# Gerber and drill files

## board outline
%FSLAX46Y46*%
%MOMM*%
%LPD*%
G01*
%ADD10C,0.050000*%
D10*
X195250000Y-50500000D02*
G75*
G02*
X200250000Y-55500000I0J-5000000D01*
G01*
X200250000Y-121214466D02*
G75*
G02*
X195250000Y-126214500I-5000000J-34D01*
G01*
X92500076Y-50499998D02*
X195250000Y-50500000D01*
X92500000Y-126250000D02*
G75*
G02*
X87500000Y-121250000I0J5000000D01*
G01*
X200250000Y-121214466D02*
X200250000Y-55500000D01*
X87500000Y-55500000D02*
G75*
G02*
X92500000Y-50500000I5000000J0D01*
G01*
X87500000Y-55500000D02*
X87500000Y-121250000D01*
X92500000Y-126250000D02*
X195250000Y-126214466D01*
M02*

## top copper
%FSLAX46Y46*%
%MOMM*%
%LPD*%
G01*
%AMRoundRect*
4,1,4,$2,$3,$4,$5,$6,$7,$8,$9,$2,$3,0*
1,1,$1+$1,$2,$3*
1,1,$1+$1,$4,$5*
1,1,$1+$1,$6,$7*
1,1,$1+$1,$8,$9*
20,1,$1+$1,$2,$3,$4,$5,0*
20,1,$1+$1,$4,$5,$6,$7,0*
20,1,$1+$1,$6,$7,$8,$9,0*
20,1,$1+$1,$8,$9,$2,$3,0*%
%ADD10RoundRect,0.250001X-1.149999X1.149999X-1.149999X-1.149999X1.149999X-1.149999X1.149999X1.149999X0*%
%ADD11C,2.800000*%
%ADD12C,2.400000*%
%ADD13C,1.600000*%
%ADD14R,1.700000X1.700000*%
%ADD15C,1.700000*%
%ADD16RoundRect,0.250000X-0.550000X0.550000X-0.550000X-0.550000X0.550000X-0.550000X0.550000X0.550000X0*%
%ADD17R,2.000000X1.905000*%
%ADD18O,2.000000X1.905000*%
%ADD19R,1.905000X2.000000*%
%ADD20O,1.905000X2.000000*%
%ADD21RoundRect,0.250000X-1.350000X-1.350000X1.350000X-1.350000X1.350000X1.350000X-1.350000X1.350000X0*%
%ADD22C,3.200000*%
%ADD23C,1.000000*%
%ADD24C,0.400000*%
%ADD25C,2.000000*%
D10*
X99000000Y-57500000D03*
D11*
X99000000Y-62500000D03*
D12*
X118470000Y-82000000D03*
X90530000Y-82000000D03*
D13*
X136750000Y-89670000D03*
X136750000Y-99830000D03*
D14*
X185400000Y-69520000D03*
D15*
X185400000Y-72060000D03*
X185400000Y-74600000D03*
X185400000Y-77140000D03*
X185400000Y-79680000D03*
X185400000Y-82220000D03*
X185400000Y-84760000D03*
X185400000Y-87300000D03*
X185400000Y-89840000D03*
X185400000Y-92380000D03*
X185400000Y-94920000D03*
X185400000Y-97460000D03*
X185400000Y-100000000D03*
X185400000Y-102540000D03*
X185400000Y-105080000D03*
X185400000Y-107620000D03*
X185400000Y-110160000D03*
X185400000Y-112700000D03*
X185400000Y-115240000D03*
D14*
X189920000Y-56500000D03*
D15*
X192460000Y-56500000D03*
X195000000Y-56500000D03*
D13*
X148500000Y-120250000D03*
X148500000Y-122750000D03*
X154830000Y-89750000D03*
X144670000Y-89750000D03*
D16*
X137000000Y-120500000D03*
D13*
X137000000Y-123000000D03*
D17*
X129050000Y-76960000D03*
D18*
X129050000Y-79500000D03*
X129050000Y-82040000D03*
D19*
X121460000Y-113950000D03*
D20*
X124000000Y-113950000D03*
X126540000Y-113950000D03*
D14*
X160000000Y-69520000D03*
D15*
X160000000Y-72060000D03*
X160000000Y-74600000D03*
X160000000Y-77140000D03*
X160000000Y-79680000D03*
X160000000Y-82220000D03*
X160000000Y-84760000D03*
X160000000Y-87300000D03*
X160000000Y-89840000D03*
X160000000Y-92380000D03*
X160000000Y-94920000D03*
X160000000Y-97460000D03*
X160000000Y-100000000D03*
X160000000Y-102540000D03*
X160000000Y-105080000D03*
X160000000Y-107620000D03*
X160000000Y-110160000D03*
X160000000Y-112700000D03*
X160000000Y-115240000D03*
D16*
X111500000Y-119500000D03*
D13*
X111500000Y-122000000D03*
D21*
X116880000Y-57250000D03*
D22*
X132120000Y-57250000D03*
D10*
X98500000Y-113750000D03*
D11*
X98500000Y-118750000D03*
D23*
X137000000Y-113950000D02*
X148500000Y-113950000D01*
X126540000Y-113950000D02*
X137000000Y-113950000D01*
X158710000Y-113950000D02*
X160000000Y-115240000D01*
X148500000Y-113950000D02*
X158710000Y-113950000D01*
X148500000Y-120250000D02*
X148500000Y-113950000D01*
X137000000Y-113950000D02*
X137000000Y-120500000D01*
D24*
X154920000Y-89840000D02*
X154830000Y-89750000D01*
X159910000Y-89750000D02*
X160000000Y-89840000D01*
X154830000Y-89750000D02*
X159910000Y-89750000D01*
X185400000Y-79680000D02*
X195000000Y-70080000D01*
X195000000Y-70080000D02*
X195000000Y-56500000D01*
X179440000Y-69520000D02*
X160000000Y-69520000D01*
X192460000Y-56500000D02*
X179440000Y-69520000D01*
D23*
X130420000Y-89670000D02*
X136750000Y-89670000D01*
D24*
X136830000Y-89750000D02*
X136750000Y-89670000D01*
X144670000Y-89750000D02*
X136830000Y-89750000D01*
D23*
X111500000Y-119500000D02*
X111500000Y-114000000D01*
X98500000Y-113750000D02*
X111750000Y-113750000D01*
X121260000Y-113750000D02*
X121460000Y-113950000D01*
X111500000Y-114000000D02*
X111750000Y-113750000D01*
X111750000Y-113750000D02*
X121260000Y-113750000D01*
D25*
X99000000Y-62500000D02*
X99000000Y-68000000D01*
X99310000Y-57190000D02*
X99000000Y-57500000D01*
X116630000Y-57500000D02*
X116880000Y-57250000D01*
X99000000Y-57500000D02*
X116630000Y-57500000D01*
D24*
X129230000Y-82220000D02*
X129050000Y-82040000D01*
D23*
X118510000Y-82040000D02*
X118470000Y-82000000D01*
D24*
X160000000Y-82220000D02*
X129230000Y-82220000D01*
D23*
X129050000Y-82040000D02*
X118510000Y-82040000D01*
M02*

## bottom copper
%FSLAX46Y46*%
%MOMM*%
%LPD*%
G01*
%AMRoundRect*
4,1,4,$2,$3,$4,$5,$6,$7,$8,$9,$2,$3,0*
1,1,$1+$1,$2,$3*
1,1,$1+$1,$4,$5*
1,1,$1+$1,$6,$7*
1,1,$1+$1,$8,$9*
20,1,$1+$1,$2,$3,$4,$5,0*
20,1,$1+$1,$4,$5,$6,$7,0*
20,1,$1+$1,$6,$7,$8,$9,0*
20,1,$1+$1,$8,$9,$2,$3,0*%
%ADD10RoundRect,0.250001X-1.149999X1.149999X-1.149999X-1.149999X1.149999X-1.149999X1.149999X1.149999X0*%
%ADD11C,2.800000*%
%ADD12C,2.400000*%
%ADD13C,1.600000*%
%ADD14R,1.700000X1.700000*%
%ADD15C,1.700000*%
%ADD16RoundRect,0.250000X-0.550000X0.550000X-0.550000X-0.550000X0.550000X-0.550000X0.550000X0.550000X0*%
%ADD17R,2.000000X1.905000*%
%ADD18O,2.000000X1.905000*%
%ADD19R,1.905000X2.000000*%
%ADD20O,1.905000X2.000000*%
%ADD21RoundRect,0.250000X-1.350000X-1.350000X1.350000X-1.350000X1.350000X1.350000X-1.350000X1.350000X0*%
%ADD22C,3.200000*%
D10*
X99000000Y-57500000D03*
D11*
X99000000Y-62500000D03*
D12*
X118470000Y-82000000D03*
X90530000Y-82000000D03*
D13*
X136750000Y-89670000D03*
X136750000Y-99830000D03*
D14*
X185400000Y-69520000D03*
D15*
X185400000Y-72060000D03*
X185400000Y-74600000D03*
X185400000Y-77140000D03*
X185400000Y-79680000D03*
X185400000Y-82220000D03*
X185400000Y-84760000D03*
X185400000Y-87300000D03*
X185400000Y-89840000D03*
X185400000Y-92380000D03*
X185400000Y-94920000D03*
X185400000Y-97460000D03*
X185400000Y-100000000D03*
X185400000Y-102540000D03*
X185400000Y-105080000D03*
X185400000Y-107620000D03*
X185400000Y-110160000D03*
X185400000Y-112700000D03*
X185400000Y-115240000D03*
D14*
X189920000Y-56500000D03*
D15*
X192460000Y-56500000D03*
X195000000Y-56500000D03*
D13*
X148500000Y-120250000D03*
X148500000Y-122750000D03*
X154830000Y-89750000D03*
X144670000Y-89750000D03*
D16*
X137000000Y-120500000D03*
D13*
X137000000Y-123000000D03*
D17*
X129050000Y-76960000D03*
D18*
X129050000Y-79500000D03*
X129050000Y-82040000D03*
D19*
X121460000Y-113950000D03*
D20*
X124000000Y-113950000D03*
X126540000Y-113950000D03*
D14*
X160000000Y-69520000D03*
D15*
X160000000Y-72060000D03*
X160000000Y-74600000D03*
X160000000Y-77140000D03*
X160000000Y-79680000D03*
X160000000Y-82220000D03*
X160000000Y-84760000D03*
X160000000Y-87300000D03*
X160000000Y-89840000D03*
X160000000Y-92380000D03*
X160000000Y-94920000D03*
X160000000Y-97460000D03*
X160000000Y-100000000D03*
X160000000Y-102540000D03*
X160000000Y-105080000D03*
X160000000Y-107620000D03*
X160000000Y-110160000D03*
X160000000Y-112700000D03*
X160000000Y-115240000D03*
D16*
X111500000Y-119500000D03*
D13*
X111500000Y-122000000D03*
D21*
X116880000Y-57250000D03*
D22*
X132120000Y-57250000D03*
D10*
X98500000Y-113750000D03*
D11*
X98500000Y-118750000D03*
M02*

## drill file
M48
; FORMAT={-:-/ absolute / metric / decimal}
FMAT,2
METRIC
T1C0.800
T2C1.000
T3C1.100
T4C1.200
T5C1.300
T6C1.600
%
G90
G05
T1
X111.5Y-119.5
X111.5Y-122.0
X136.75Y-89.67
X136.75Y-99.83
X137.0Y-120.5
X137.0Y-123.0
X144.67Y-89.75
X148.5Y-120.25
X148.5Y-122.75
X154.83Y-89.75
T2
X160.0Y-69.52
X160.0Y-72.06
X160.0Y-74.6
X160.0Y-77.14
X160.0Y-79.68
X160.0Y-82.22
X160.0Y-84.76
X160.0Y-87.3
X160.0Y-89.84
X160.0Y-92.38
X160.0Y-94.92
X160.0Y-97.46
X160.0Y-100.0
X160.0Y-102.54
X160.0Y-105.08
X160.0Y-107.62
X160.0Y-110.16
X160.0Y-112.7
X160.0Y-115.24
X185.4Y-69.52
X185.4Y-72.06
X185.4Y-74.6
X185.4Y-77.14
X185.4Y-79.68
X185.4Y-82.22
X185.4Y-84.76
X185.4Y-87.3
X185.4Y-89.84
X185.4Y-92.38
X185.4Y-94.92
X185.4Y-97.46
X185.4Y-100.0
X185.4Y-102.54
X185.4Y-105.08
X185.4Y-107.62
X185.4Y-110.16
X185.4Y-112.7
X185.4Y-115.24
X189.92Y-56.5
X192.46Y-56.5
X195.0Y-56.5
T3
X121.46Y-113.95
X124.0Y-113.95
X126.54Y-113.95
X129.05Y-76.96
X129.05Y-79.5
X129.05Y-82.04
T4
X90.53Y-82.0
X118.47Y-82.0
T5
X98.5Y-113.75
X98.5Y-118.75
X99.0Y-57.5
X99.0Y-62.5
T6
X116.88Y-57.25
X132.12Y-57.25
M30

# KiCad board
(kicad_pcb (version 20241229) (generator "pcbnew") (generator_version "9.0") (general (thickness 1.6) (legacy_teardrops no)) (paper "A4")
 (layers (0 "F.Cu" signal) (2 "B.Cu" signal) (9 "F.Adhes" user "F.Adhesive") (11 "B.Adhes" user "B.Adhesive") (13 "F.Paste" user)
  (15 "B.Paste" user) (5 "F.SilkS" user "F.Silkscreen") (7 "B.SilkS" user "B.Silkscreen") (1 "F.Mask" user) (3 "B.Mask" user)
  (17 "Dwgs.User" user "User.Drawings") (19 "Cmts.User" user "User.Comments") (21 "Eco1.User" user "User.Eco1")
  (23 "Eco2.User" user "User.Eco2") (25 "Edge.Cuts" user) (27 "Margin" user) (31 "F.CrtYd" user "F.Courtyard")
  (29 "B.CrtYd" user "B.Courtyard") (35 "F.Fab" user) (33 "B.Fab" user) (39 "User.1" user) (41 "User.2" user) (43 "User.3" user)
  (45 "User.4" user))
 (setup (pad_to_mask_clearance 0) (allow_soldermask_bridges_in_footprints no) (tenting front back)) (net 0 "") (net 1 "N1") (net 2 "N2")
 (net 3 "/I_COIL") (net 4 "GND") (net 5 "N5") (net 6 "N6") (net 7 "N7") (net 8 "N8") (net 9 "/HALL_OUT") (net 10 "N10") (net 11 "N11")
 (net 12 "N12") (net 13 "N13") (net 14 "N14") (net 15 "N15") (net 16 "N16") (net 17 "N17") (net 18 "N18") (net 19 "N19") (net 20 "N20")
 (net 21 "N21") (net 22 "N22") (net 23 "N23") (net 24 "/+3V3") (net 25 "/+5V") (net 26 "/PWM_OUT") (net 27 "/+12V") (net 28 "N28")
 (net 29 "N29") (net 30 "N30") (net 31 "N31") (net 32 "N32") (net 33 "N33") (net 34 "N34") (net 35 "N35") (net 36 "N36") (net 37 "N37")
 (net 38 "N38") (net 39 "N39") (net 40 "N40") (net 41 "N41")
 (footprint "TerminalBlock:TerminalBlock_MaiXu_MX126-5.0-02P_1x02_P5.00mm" (layer "F.Cu") (at 99 57.5 -90)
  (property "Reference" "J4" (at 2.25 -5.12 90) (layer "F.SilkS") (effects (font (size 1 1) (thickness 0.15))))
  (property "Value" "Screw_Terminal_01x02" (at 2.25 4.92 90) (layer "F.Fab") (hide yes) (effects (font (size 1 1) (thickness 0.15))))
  (pad "1" thru_hole roundrect (at 0 0 270) (size 2.8 2.8) (drill 1.3) (layers "*.Cu" "*.Mask") (remove_unused_layers no)
   (roundrect_rratio 0.089286) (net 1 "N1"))
  (pad "2" thru_hole circle (at 5 0 270) (size 2.8 2.8) (drill 1.3) (layers "*.Cu" "*.Mask") (remove_unused_layers no) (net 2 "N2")))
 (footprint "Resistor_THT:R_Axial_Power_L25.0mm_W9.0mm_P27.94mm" (layer "F.Cu") (at 118.47 82 180)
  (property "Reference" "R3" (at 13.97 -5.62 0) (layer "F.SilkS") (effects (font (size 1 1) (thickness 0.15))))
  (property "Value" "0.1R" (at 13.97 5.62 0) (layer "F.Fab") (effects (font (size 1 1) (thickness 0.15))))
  (pad "1" thru_hole circle (at 0 0 180) (size 2.4 2.4) (drill 1.2) (layers "*.Cu" "*.Mask") (remove_unused_layers no) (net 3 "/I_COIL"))
  (pad "2" thru_hole circle (at 27.94 0 180) (size 2.4 2.4) (drill 1.2) (layers "*.Cu" "*.Mask") (remove_unused_layers no) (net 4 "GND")))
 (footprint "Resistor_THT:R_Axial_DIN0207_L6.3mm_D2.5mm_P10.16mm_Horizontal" (layer "F.Cu") (at 136.75 89.67 -90)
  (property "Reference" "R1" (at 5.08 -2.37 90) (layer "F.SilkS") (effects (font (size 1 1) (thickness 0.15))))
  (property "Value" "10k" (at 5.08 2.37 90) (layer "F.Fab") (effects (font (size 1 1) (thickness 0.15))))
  (pad "1" thru_hole circle (at 0 0 270) (size 1.6 1.6) (drill 0.8) (layers "*.Cu" "*.Mask") (remove_unused_layers no) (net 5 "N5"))
  (pad "2" thru_hole circle (at 10.16 0 270) (size 1.6 1.6) (drill 0.8) (layers "*.Cu" "*.Mask") (remove_unused_layers no) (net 4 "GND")))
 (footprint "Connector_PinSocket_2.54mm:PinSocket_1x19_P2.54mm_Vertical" (layer "F.Cu") (at 185.4 69.52)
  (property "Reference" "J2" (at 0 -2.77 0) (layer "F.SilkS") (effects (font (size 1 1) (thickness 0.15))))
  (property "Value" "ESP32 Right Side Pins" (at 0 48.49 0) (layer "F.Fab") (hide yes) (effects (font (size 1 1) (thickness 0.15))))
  (pad "1" thru_hole rect (at 0 0) (size 1.7 1.7) (drill 1) (layers "*.Cu" "*.Mask") (remove_unused_layers no) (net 4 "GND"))
  (pad "2" thru_hole circle (at 0 2.54) (size 1.7 1.7) (drill 1) (layers "*.Cu" "*.Mask") (remove_unused_layers no) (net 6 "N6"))
  (pad "3" thru_hole circle (at 0 5.08) (size 1.7 1.7) (drill 1) (layers "*.Cu" "*.Mask") (remove_unused_layers no) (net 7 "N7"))
  (pad "4" thru_hole circle (at 0 7.62) (size 1.7 1.7) (drill 1) (layers "*.Cu" "*.Mask") (remove_unused_layers no) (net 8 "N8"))
  (pad "5" thru_hole circle (at 0 10.16) (size 1.7 1.7) (drill 1) (layers "*.Cu" "*.Mask") (remove_unused_layers no) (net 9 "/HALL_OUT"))
  (pad "6" thru_hole circle (at 0 12.7) (size 1.7 1.7) (drill 1) (layers "*.Cu" "*.Mask") (remove_unused_layers no) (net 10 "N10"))
  (pad "7" thru_hole circle (at 0 15.24) (size 1.7 1.7) (drill 1) (layers "*.Cu" "*.Mask") (remove_unused_layers no) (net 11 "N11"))
  (pad "8" thru_hole circle (at 0 17.78) (size 1.7 1.7) (drill 1) (layers "*.Cu" "*.Mask") (remove_unused_layers no) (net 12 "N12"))
  (pad "9" thru_hole circle (at 0 20.32) (size 1.7 1.7) (drill 1) (layers "*.Cu" "*.Mask") (remove_unused_layers no) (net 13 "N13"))
  (pad "10" thru_hole circle (at 0 22.86) (size 1.7 1.7) (drill 1) (layers "*.Cu" "*.Mask") (remove_unused_layers no) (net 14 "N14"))
  (pad "11" thru_hole circle (at 0 25.4) (size 1.7 1.7) (drill 1) (layers "*.Cu" "*.Mask") (remove_unused_layers no) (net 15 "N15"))
  (pad "12" thru_hole circle (at 0 27.94) (size 1.7 1.7) (drill 1) (layers "*.Cu" "*.Mask") (remove_unused_layers no) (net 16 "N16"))
  (pad "13" thru_hole circle (at 0 30.48) (size 1.7 1.7) (drill 1) (layers "*.Cu" "*.Mask") (remove_unused_layers no) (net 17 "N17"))
  (pad "14" thru_hole circle (at 0 33.02) (size 1.7 1.7) (drill 1) (layers "*.Cu" "*.Mask") (remove_unused_layers no) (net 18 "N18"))
  (pad "15" thru_hole circle (at 0 35.56) (size 1.7 1.7) (drill 1) (layers "*.Cu" "*.Mask") (remove_unused_layers no) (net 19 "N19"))
  (pad "16" thru_hole circle (at 0 38.1) (size 1.7 1.7) (drill 1) (layers "*.Cu" "*.Mask") (remove_unused_layers no) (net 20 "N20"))
  (pad "17" thru_hole circle (at 0 40.64) (size 1.7 1.7) (drill 1) (layers "*.Cu" "*.Mask") (remove_unused_layers no) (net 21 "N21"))
  (pad "18" thru_hole circle (at 0 43.18) (size 1.7 1.7) (drill 1) (layers "*.Cu" "*.Mask") (remove_unused_layers no) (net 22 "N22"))
  (pad "19" thru_hole circle (at 0 45.72) (size 1.7 1.7) (drill 1) (layers "*.Cu" "*.Mask") (remove_unused_layers no) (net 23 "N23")))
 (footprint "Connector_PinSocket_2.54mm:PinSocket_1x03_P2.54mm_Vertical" (layer "F.Cu") (at 189.92 56.5 90)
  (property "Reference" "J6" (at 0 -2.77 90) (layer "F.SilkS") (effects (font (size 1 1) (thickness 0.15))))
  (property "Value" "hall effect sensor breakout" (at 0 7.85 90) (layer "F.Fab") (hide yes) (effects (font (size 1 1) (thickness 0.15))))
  (pad "1" thru_hole rect (at 0 0 90) (size 1.7 1.7) (drill 1) (layers "*.Cu" "*.Mask") (remove_unused_layers no) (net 4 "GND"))
  (pad "2" thru_hole circle (at 0 2.54 90) (size 1.7 1.7) (drill 1) (layers "*.Cu" "*.Mask") (remove_unused_layers no) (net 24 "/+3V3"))
  (pad "3" thru_hole circle (at 0 5.08 90) (size 1.7 1.7) (drill 1) (layers "*.Cu" "*.Mask") (remove_unused_layers no) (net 9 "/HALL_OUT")))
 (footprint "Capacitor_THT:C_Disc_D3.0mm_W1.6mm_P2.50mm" (layer "F.Cu") (at 148.5 120.25 -90)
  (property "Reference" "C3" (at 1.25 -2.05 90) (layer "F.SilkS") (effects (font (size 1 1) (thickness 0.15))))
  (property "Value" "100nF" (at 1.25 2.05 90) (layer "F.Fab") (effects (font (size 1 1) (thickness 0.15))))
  (pad "1" thru_hole circle (at 0 0 270) (size 1.6 1.6) (drill 0.8) (layers "*.Cu" "*.Mask") (remove_unused_layers no) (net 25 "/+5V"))
  (pad "2" thru_hole circle (at 2.5 0 270) (size 1.6 1.6) (drill 0.8) (layers "*.Cu" "*.Mask") (remove_unused_layers no) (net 4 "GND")))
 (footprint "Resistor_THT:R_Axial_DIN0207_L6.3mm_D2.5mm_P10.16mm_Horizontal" (layer "F.Cu") (at 154.83 89.75 180)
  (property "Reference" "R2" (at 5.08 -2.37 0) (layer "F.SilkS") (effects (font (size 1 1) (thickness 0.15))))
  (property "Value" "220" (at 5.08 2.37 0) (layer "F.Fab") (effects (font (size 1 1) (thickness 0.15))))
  (pad "1" thru_hole circle (at 0 0 180) (size 1.6 1.6) (drill 0.8) (layers "*.Cu" "*.Mask") (remove_unused_layers no) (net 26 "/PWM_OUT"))
  (pad "2" thru_hole circle (at 10.16 0 180) (size 1.6 1.6) (drill 0.8) (layers "*.Cu" "*.Mask") (remove_unused_layers no) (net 5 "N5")))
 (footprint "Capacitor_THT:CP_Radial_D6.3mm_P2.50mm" (layer "F.Cu") (at 137 120.5 -90)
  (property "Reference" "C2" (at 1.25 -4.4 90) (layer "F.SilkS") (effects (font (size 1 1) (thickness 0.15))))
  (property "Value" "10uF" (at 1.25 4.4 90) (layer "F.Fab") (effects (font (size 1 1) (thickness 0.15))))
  (pad "1" thru_hole roundrect (at 0 0 270) (size 1.6 1.6) (drill 0.8) (layers "*.Cu" "*.Mask") (remove_unused_layers no)
   (roundrect_rratio 0.15625) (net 25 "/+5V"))
  (pad "2" thru_hole circle (at 2.5 0 270) (size 1.6 1.6) (drill 0.8) (layers "*.Cu" "*.Mask") (remove_unused_layers no) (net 4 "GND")))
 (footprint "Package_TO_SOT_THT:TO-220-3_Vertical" (layer "F.Cu") (at 129.05 76.96 -90)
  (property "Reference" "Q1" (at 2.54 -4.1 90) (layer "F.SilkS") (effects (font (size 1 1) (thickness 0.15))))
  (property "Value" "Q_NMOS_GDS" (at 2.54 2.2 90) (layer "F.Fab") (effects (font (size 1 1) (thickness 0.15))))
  (pad "1" thru_hole rect (at 0 0 270) (size 1.905 2) (drill 1.1) (layers "*.Cu" "*.Mask") (remove_unused_layers no) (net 5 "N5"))
  (pad "2" thru_hole oval (at 2.54 0 270) (size 1.905 2) (drill 1.1) (layers "*.Cu" "*.Mask") (remove_unused_layers no) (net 2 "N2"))
  (pad "3" thru_hole oval (at 5.08 0 270) (size 1.905 2) (drill 1.1) (layers "*.Cu" "*.Mask") (remove_unused_layers no) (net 3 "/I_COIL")))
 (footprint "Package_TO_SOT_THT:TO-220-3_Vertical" (layer "F.Cu") (at 121.46 113.95)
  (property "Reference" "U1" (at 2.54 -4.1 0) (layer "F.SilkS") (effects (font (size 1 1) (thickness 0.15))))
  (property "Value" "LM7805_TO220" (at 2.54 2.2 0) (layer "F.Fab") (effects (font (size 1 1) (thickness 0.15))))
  (pad "1" thru_hole rect (at 0 0) (size 1.905 2) (drill 1.1) (layers "*.Cu" "*.Mask") (remove_unused_layers no) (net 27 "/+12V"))
  (pad "2" thru_hole oval (at 2.54 0) (size 1.905 2) (drill 1.1) (layers "*.Cu" "*.Mask") (remove_unused_layers no) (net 4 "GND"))
  (pad "3" thru_hole oval (at 5.08 0) (size 1.905 2) (drill 1.1) (layers "*.Cu" "*.Mask") (remove_unused_layers no) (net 25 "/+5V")))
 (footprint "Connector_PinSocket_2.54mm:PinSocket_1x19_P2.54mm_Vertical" (layer "F.Cu") (at 160 69.52)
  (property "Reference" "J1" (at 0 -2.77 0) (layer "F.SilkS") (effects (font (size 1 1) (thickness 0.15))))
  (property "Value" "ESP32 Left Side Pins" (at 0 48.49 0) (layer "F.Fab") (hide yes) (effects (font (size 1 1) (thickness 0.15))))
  (pad "1" thru_hole rect (at 0 0) (size 1.7 1.7) (drill 1) (layers "*.Cu" "*.Mask") (remove_unused_layers no) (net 24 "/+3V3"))
  (pad "2" thru_hole circle (at 0 2.54) (size 1.7 1.7) (drill 1) (layers "*.Cu" "*.Mask") (remove_unused_layers no) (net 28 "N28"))
  (pad "3" thru_hole circle (at 0 5.08) (size 1.7 1.7) (drill 1) (layers "*.Cu" "*.Mask") (remove_unused_layers no) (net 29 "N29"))
  (pad "4" thru_hole circle (at 0 7.62) (size 1.7 1.7) (drill 1) (layers "*.Cu" "*.Mask") (remove_unused_layers no) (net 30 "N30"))
  (pad "5" thru_hole circle (at 0 10.16) (size 1.7 1.7) (drill 1) (layers "*.Cu" "*.Mask") (remove_unused_layers no) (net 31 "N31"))
  (pad "6" thru_hole circle (at 0 12.7) (size 1.7 1.7) (drill 1) (layers "*.Cu" "*.Mask") (remove_unused_layers no) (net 3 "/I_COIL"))
  (pad "7" thru_hole circle (at 0 15.24) (size 1.7 1.7) (drill 1) (layers "*.Cu" "*.Mask") (remove_unused_layers no) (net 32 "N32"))
  (pad "8" thru_hole circle (at 0 17.78) (size 1.7 1.7) (drill 1) (layers "*.Cu" "*.Mask") (remove_unused_layers no) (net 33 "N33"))
  (pad "9" thru_hole circle (at 0 20.32) (size 1.7 1.7) (drill 1) (layers "*.Cu" "*.Mask") (remove_unused_layers no) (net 26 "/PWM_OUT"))
  (pad "10" thru_hole circle (at 0 22.86) (size 1.7 1.7) (drill 1) (layers "*.Cu" "*.Mask") (remove_unused_layers no) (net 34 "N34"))
  (pad "11" thru_hole circle (at 0 25.4) (size 1.7 1.7) (drill 1) (layers "*.Cu" "*.Mask") (remove_unused_layers no) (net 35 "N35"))
  (pad "12" thru_hole circle (at 0 27.94) (size 1.7 1.7) (drill 1) (layers "*.Cu" "*.Mask") (remove_unused_layers no) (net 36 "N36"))
  (pad "13" thru_hole circle (at 0 30.48) (size 1.7 1.7) (drill 1) (layers "*.Cu" "*.Mask") (remove_unused_layers no) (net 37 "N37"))
  (pad "14" thru_hole circle (at 0 33.02) (size 1.7 1.7) (drill 1) (layers "*.Cu" "*.Mask") (remove_unused_layers no) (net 4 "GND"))
  (pad "15" thru_hole circle (at 0 35.56) (size 1.7 1.7) (drill 1) (layers "*.Cu" "*.Mask") (remove_unused_layers no) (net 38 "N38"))
  (pad "16" thru_hole circle (at 0 38.1) (size 1.7 1.7) (drill 1) (layers "*.Cu" "*.Mask") (remove_unused_layers no) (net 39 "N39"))
  (pad "17" thru_hole circle (at 0 40.64) (size 1.7 1.7) (drill 1) (layers "*.Cu" "*.Mask") (remove_unused_layers no) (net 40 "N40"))
  (pad "18" thru_hole circle (at 0 43.18) (size 1.7 1.7) (drill 1) (layers "*.Cu" "*.Mask") (remove_unused_layers no) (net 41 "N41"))
  (pad "19" thru_hole circle (at 0 45.72) (size 1.7 1.7) (drill 1) (layers "*.Cu" "*.Mask") (remove_unused_layers no) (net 25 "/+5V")))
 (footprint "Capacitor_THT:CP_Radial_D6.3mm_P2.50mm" (layer "F.Cu") (at 111.5 119.5 -90)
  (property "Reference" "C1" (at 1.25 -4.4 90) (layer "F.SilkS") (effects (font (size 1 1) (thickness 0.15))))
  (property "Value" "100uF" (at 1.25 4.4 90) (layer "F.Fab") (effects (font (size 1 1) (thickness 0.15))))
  (pad "1" thru_hole roundrect (at 0 0 270) (size 1.6 1.6) (drill 0.8) (layers "*.Cu" "*.Mask") (remove_unused_layers no)
   (roundrect_rratio 0.15625) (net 27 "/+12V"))
  (pad "2" thru_hole circle (at 2.5 0 270) (size 1.6 1.6) (drill 0.8) (layers "*.Cu" "*.Mask") (remove_unused_layers no) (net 4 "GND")))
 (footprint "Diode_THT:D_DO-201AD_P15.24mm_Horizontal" (layer "F.Cu") (at 116.88 57.25)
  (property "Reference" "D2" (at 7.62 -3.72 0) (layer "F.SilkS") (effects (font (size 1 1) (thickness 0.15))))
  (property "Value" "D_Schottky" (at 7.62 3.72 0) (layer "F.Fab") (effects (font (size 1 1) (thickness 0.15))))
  (pad "1" thru_hole roundrect (at 0 0) (size 3.2 3.2) (drill 1.6) (layers "*.Cu" "*.Mask") (remove_unused_layers no)
   (roundrect_rratio 0.078125) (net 1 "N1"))
  (pad "2" thru_hole circle (at 15.24 0) (size 3.2 3.2) (drill 1.6) (layers "*.Cu" "*.Mask") (remove_unused_layers no) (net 2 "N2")))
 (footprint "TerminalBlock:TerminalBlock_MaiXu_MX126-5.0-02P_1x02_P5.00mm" (layer "F.Cu") (at 98.5 113.75 -90)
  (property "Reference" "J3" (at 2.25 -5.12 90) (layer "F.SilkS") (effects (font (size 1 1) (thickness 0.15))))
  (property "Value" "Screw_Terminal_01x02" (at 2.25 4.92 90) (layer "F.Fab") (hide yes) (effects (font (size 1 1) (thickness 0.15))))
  (pad "1" thru_hole roundrect (at 0 0 270) (size 2.8 2.8) (drill 1.3) (layers "*.Cu" "*.Mask") (remove_unused_layers no)
   (roundrect_rratio 0.089286) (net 27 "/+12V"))
  (pad "2" thru_hole circle (at 5 0 270) (size 2.8 2.8) (drill 1.3) (layers "*.Cu" "*.Mask") (remove_unused_layers no) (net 4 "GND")))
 (gr_arc (start 195.25 50.5) (mid 198.785534 51.964466) (end 200.25 55.5) (stroke (width 0.05) (type default)) (layer "Edge.Cuts"))
 (gr_arc (start 200.25 121.214466) (mid 198.785534 124.75) (end 195.25 126.214466) (stroke (width 0.05) (type default)) (layer "Edge.Cuts"))
 (gr_line (start 92.500076 50.499998) (end 195.25 50.5) (stroke (width 0.05) (type default)) (layer "Edge.Cuts"))
 (gr_arc (start 92.5 126.25) (mid 88.964466 124.785534) (end 87.5 121.25) (stroke (width 0.05) (type default)) (layer "Edge.Cuts"))
 (gr_line (start 200.25 121.214466) (end 200.25 55.5) (stroke (width 0.05) (type default)) (layer "Edge.Cuts"))
 (gr_arc (start 87.5 55.5) (mid 88.964466 51.964466) (end 92.5 50.5) (stroke (width 0.05) (type default)) (layer "Edge.Cuts"))
 (gr_line (start 87.5 55.5) (end 87.5 121.25) (stroke (width 0.05) (type default)) (layer "Edge.Cuts"))
 (gr_line (start 92.5 126.25) (end 195.25 126.214466) (stroke (width 0.05) (type default)) (layer "Edge.Cuts"))
 (segment (start 137 113.95) (end 148.5 113.95) (width 1) (layer "F.Cu") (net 25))
 (segment (start 126.54 113.95) (end 137 113.95) (width 1) (layer "F.Cu") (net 25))
 (segment (start 158.71 113.95) (end 160 115.24) (width 1) (layer "F.Cu") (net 25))
 (segment (start 148.5 113.95) (end 158.71 113.95) (width 1) (layer "F.Cu") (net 25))
 (segment (start 148.5 120.25) (end 148.5 113.95) (width 1) (layer "F.Cu") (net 25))
 (segment (start 137 113.95) (end 137 120.5) (width 1) (layer "F.Cu") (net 25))
 (segment (start 154.92 89.84) (end 154.83 89.75) (width 0.4) (layer "F.Cu") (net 26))
 (segment (start 159.91 89.75) (end 160 89.84) (width 0.4) (layer "F.Cu") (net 26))
 (segment (start 154.83 89.75) (end 159.91 89.75) (width 0.4) (layer "F.Cu") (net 26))
 (segment (start 185.4 79.68) (end 195 70.08) (width 0.4) (layer "F.Cu") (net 9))
 (segment (start 195 70.08) (end 195 56.5) (width 0.4) (layer "F.Cu") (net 9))
 (segment (start 179.44 69.52) (end 160 69.52) (width 0.4) (layer "F.Cu") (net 24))
 (segment (start 192.46 56.5) (end 179.44 69.52) (width 0.4) (layer "F.Cu") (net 24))
 (segment (start 130.42 89.67) (end 136.75 89.67) (width 1) (layer "F.Cu") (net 5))
 (segment (start 136.83 89.75) (end 136.75 89.67) (width 0.4) (layer "F.Cu") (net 5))
 (segment (start 144.67 89.75) (end 136.83 89.75) (width 0.4) (layer "F.Cu") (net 5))
 (segment (start 111.5 119.5) (end 111.5 114) (width 1) (layer "F.Cu") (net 27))
 (segment (start 98.5 113.75) (end 111.75 113.75) (width 1) (layer "F.Cu") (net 27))
 (segment (start 121.26 113.75) (end 121.46 113.95) (width 1) (layer "F.Cu") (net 27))
 (segment (start 111.5 114) (end 111.75 113.75) (width 1) (layer "F.Cu") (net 27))
 (segment (start 111.75 113.75) (end 121.26 113.75) (width 1) (layer "F.Cu") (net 27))
 (segment (start 99 62.5) (end 99 68) (width 2) (layer "F.Cu") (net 2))
 (segment (start 99.31 57.19) (end 99 57.5) (width 2) (layer "F.Cu") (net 1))
 (segment (start 116.63 57.5) (end 116.88 57.25) (width 2) (layer "F.Cu") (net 1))
 (segment (start 99 57.5) (end 116.63 57.5) (width 2) (layer "F.Cu") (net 1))
 (segment (start 129.23 82.22) (end 129.05 82.04) (width 0.4) (layer "F.Cu") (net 3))
 (segment (start 118.51 82.04) (end 118.47 82) (width 1) (layer "F.Cu") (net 3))
 (segment (start 160 82.22) (end 129.23 82.22) (width 0.4) (layer "F.Cu") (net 3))
 (segment (start 129.05 82.04) (end 118.51 82.04) (width 1) (layer "F.Cu") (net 3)))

